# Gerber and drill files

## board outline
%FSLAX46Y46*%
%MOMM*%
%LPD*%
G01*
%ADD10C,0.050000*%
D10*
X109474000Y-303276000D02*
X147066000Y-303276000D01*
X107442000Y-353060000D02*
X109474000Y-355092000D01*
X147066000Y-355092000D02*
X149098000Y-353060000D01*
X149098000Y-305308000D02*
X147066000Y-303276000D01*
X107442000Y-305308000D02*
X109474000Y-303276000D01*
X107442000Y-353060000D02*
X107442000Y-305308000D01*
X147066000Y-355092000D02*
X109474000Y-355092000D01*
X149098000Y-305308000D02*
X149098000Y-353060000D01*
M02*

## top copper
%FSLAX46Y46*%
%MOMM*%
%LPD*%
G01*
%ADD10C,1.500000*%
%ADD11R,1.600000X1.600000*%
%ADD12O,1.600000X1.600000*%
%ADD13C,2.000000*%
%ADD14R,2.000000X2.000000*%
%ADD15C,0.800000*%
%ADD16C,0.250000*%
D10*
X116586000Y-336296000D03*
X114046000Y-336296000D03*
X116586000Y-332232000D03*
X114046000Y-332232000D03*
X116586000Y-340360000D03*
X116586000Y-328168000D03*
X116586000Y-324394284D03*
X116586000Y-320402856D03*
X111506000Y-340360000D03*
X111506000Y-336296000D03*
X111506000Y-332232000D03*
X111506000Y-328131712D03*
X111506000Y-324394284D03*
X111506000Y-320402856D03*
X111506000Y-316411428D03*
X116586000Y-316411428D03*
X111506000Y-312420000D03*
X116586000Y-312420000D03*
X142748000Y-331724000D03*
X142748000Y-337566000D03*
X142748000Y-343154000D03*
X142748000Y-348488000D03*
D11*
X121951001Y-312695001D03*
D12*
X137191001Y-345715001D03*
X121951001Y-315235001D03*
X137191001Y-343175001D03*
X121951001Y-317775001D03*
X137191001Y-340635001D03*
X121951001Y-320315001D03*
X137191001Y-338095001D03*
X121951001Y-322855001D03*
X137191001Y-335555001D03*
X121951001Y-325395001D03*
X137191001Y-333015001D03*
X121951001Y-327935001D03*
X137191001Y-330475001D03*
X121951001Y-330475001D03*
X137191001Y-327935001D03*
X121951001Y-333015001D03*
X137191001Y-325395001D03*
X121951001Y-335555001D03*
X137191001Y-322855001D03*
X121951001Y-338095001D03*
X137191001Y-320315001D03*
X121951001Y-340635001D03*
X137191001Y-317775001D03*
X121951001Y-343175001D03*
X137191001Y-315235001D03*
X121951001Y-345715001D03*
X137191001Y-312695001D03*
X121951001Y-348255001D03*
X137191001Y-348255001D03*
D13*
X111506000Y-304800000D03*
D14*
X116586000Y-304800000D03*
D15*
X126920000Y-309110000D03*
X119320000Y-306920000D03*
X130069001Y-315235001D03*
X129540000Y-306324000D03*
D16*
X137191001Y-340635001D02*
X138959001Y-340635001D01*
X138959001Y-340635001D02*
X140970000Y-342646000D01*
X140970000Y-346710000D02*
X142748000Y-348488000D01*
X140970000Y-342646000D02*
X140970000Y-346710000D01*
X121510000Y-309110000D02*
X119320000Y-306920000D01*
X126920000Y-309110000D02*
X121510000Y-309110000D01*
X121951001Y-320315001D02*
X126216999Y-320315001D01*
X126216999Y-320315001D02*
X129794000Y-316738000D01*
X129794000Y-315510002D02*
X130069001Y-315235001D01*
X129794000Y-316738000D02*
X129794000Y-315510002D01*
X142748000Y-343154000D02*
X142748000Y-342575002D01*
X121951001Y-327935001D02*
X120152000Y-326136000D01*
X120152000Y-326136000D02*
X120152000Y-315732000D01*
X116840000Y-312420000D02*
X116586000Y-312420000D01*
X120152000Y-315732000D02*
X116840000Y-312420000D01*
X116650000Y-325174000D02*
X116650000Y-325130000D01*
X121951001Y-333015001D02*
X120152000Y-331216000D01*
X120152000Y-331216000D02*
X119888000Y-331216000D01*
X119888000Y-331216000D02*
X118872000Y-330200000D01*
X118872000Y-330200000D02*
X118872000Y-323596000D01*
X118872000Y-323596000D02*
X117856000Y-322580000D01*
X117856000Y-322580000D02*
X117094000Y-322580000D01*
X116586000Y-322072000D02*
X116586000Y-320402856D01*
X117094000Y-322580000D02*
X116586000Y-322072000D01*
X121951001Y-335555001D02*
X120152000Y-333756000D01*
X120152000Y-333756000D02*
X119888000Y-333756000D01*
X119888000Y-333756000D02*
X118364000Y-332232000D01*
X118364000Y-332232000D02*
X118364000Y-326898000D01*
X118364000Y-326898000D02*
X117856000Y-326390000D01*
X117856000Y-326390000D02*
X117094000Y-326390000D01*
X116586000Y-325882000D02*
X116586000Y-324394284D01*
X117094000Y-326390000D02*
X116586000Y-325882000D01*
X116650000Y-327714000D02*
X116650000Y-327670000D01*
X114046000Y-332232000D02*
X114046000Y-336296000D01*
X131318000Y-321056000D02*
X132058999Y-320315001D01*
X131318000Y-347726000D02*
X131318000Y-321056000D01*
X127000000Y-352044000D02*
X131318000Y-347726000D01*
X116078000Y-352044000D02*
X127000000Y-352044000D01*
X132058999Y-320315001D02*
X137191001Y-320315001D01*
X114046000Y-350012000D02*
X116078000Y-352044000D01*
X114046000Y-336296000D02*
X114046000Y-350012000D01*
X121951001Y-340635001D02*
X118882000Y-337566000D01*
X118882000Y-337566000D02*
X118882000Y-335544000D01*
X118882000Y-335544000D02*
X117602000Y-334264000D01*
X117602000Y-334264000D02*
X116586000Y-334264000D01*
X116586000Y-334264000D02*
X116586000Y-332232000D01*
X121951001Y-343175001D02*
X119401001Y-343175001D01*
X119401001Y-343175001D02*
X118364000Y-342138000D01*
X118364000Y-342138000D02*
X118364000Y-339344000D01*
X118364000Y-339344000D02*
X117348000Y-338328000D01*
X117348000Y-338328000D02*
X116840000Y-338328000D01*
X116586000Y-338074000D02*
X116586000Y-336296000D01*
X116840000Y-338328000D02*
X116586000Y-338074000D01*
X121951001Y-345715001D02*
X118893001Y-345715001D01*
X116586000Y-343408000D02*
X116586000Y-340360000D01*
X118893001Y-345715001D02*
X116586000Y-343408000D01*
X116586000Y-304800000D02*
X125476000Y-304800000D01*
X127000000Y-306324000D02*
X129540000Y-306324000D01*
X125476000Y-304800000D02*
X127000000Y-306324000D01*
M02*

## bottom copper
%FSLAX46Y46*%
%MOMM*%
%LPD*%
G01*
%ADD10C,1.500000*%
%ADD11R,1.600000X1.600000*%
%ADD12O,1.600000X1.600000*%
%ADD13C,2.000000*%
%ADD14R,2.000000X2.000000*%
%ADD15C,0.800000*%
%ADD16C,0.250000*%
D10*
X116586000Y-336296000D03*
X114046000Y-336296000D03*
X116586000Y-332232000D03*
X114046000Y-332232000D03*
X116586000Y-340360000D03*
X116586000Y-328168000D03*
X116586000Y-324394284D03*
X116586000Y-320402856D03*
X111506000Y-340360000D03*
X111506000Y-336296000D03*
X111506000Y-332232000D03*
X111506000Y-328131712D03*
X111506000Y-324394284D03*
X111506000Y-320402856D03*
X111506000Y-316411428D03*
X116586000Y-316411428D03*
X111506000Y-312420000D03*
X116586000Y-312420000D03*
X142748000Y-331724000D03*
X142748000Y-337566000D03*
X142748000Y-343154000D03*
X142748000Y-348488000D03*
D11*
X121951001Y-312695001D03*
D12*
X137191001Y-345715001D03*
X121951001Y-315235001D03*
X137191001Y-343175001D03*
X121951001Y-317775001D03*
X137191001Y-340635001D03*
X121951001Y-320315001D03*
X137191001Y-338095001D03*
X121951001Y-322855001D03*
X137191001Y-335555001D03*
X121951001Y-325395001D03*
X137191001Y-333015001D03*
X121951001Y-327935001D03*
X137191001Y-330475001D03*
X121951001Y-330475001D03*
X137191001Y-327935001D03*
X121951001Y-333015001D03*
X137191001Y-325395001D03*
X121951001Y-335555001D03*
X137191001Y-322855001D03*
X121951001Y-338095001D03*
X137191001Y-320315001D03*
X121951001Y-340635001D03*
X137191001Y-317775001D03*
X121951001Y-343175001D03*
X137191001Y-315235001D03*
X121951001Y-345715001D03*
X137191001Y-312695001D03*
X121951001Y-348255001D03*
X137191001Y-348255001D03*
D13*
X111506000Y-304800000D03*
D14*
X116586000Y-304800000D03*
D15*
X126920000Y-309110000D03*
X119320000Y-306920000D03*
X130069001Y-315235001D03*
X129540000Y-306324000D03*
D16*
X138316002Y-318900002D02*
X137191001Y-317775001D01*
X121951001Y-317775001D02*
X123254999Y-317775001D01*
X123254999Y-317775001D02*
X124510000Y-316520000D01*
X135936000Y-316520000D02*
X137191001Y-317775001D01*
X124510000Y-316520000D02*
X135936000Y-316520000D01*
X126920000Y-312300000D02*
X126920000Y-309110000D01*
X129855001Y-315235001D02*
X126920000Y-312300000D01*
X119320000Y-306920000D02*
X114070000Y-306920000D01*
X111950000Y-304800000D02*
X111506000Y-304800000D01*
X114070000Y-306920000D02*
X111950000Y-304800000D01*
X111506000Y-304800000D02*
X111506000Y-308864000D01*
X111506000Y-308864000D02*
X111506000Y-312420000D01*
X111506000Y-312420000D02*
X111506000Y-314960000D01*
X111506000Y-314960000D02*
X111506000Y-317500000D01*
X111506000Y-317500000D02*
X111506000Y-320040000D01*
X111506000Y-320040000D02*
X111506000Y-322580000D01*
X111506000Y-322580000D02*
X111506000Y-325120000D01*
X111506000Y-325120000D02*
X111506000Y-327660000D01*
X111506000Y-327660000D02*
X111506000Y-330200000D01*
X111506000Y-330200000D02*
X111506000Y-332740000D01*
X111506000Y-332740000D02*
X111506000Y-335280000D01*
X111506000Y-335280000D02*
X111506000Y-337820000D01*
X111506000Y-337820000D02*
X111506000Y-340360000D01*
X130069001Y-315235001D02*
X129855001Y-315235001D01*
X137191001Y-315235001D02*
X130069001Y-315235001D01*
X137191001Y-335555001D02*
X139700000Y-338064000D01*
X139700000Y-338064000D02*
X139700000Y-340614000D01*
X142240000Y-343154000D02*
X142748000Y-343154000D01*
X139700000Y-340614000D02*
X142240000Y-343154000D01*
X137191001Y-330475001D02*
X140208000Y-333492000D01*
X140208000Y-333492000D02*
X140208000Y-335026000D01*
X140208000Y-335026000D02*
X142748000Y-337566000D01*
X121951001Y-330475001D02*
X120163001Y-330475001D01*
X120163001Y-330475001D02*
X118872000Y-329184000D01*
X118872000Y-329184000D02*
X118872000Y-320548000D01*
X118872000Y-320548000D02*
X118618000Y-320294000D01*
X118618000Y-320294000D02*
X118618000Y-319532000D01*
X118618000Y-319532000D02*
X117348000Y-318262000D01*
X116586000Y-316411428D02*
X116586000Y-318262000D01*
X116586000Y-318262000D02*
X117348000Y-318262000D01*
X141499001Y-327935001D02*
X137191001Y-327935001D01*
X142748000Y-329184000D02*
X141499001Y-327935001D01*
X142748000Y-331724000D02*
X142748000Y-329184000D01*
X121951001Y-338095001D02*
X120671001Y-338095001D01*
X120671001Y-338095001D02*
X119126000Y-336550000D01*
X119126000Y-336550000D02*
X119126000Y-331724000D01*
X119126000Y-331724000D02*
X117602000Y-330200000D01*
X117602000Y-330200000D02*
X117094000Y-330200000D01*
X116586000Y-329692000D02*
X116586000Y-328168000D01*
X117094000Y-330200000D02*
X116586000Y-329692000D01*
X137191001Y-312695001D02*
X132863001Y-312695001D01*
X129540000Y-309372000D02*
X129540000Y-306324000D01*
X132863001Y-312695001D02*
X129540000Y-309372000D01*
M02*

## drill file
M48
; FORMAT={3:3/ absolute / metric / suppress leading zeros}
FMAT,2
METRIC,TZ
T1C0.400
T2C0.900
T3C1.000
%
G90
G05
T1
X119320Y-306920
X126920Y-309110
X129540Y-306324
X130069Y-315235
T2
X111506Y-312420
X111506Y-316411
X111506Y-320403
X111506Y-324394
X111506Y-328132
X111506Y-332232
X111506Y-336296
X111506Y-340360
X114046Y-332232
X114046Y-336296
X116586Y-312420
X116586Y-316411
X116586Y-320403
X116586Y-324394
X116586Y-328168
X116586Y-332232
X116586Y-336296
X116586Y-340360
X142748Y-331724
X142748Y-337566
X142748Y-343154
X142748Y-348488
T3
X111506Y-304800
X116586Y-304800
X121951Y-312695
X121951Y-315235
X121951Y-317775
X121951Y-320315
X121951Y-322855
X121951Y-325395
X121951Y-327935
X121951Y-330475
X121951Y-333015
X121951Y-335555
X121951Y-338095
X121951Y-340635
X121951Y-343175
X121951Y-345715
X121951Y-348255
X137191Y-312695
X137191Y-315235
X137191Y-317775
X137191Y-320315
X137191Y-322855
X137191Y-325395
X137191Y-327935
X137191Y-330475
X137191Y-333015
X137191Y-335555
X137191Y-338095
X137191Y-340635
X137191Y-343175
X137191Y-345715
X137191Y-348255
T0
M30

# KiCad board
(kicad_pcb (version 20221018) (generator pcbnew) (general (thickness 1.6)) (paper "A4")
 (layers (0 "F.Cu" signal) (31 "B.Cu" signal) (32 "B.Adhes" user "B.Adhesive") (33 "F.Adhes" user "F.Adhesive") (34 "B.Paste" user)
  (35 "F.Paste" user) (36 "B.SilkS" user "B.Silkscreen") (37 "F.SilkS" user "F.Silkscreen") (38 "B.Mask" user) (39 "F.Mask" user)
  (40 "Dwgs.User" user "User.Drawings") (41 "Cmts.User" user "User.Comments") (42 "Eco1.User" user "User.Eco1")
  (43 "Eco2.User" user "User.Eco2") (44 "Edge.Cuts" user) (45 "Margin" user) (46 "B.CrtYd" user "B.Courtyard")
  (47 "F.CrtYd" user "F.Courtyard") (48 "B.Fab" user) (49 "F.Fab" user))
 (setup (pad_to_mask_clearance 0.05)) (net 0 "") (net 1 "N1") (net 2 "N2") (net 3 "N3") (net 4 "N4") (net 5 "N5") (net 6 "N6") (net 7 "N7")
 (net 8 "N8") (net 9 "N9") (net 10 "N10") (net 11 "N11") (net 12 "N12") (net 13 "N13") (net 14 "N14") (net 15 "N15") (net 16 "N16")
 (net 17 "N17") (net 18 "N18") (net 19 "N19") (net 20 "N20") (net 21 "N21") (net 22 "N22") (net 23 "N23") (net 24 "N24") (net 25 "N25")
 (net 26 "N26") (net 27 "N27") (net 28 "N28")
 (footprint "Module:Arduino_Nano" (layer "F.Cu") (at 121.951001 312.695001)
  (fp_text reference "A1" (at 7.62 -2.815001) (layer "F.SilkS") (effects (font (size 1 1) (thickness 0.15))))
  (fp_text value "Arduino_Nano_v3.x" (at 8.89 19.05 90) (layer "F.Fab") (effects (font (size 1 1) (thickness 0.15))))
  (pad "1" thru_hole rect (at 0 0) (size 1.6 1.6) (drill 1) (layers "*.Cu" "*.Mask") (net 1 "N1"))
  (pad "2" thru_hole oval (at 0 2.54) (size 1.6 1.6) (drill 1) (layers "*.Cu" "*.Mask") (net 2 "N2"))
  (pad "3" thru_hole oval (at 0 5.08) (size 1.6 1.6) (drill 1) (layers "*.Cu" "*.Mask") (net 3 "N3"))
  (pad "4" thru_hole oval (at 0 7.62) (size 1.6 1.6) (drill 1) (layers "*.Cu" "*.Mask") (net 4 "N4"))
  (pad "5" thru_hole oval (at 0 10.16) (size 1.6 1.6) (drill 1) (layers "*.Cu" "*.Mask") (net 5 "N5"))
  (pad "6" thru_hole oval (at 0 12.7) (size 1.6 1.6) (drill 1) (layers "*.Cu" "*.Mask") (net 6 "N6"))
  (pad "7" thru_hole oval (at 0 15.24) (size 1.6 1.6) (drill 1) (layers "*.Cu" "*.Mask") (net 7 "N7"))
  (pad "8" thru_hole oval (at 0 17.78) (size 1.6 1.6) (drill 1) (layers "*.Cu" "*.Mask") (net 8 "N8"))
  (pad "9" thru_hole oval (at 0 20.32) (size 1.6 1.6) (drill 1) (layers "*.Cu" "*.Mask") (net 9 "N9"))
  (pad "10" thru_hole oval (at 0 22.86) (size 1.6 1.6) (drill 1) (layers "*.Cu" "*.Mask") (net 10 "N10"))
  (pad "11" thru_hole oval (at 0 25.4) (size 1.6 1.6) (drill 1) (layers "*.Cu" "*.Mask") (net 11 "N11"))
  (pad "12" thru_hole oval (at 0 27.94) (size 1.6 1.6) (drill 1) (layers "*.Cu" "*.Mask") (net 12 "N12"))
  (pad "13" thru_hole oval (at 0 30.48) (size 1.6 1.6) (drill 1) (layers "*.Cu" "*.Mask") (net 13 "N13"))
  (pad "14" thru_hole oval (at 0 33.02) (size 1.6 1.6) (drill 1) (layers "*.Cu" "*.Mask") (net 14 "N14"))
  (pad "15" thru_hole oval (at 0 35.56) (size 1.6 1.6) (drill 1) (layers "*.Cu" "*.Mask") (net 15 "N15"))
  (pad "16" thru_hole oval (at 15.24 35.56) (size 1.6 1.6) (drill 1) (layers "*.Cu" "*.Mask") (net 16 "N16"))
  (pad "17" thru_hole oval (at 15.24 33.02) (size 1.6 1.6) (drill 1) (layers "*.Cu" "*.Mask") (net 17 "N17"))
  (pad "18" thru_hole oval (at 15.24 30.48) (size 1.6 1.6) (drill 1) (layers "*.Cu" "*.Mask") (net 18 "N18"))
  (pad "19" thru_hole oval (at 15.24 27.94) (size 1.6 1.6) (drill 1) (layers "*.Cu" "*.Mask") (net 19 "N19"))
  (pad "20" thru_hole oval (at 15.24 25.4) (size 1.6 1.6) (drill 1) (layers "*.Cu" "*.Mask") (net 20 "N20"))
  (pad "21" thru_hole oval (at 15.24 22.86) (size 1.6 1.6) (drill 1) (layers "*.Cu" "*.Mask") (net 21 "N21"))
  (pad "22" thru_hole oval (at 15.24 20.32) (size 1.6 1.6) (drill 1) (layers "*.Cu" "*.Mask") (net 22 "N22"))
  (pad "23" thru_hole oval (at 15.24 17.78) (size 1.6 1.6) (drill 1) (layers "*.Cu" "*.Mask") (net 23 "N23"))
  (pad "24" thru_hole oval (at 15.24 15.24) (size 1.6 1.6) (drill 1) (layers "*.Cu" "*.Mask") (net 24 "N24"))
  (pad "25" thru_hole oval (at 15.24 12.7) (size 1.6 1.6) (drill 1) (layers "*.Cu" "*.Mask") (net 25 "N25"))
  (pad "26" thru_hole oval (at 15.24 10.16) (size 1.6 1.6) (drill 1) (layers "*.Cu" "*.Mask") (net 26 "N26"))
  (pad "27" thru_hole oval (at 15.24 7.62) (size 1.6 1.6) (drill 1) (layers "*.Cu" "*.Mask") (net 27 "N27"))
  (pad "28" thru_hole oval (at 15.24 5.08) (size 1.6 1.6) (drill 1) (layers "*.Cu" "*.Mask") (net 3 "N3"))
  (pad "29" thru_hole oval (at 15.24 2.54) (size 1.6 1.6) (drill 1) (layers "*.Cu" "*.Mask") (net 4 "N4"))
  (pad "30" thru_hole oval (at 15.24 0) (size 1.6 1.6) (drill 1) (layers "*.Cu" "*.Mask") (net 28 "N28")))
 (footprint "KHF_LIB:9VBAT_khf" (layer "F.Cu") (at 111.506 304.8)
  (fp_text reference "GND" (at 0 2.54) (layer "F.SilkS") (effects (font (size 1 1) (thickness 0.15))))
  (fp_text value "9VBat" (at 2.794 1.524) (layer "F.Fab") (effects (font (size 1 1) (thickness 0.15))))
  (pad "1" thru_hole circle (at 0 0) (size 2 2) (drill 1) (layers "*.Cu" "*.Mask") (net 4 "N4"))
  (pad "2" thru_hole rect (at 5.08 0) (size 2 2) (drill 1) (layers "*.Cu" "*.Mask") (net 28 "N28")))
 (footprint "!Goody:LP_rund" (layer "F.Cu") (at 142.748 348.488)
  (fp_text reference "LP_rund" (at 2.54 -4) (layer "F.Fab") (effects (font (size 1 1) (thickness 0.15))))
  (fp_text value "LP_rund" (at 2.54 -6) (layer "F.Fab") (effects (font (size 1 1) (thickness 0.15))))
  (pad "1" thru_hole circle (at 0 0) (size 1.5 1.5) (drill 0.9) (layers "*.Cu" "*.Mask") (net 19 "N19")))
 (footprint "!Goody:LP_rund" (layer "F.Cu") (at 116.586 336.296)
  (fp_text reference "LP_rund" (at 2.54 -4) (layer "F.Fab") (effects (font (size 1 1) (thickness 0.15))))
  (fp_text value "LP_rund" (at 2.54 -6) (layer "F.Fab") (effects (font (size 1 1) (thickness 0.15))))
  (pad "1" thru_hole circle (at 0 0) (size 1.5 1.5) (drill 0.9) (layers "*.Cu" "*.Mask") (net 13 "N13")))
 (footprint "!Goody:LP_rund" (layer "F.Cu") (at 111.506 312.42)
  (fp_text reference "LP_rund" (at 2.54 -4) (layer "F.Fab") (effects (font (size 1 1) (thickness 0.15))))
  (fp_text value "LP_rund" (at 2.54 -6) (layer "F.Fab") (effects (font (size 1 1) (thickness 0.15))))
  (pad "1" thru_hole circle (at 0 0) (size 1.5 1.5) (drill 0.9) (layers "*.Cu" "*.Mask") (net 4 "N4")))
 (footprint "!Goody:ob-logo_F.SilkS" (layer "F.Cu") (at 130.048 329.692 90)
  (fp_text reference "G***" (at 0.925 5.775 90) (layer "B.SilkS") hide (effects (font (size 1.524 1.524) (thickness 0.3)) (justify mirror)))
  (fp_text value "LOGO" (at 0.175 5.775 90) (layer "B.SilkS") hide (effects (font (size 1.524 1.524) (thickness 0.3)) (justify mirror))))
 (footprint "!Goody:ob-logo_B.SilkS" (layer "F.Cu") (at 146.05 323.596 90)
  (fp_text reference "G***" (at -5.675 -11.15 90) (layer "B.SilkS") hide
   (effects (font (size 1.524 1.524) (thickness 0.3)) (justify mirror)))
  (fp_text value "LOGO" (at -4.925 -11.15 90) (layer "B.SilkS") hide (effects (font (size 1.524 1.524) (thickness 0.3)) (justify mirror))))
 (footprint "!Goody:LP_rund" (layer "F.Cu") (at 142.748 343.154)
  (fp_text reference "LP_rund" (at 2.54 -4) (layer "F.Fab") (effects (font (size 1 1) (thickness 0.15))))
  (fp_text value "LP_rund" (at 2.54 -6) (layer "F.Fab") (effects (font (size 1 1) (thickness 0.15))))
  (pad "1" thru_hole circle (at 0 0) (size 1.5 1.5) (drill 0.9) (layers "*.Cu" "*.Mask") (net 21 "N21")))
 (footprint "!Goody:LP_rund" (layer "F.Cu") (at 111.506 340.36)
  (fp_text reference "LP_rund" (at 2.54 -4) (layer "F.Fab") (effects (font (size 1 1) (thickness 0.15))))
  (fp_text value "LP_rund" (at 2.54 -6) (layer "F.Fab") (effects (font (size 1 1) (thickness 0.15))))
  (pad "1" thru_hole circle (at 0 0) (size 1.5 1.5) (drill 0.9) (layers "*.Cu" "*.Mask") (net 4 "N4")))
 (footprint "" (layer "F.Cu") (at 112.268 348.488)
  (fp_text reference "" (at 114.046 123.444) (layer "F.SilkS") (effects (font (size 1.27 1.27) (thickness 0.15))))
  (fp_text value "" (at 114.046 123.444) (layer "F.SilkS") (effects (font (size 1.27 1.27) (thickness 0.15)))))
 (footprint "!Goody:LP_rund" (layer "F.Cu") (at 116.586 312.42)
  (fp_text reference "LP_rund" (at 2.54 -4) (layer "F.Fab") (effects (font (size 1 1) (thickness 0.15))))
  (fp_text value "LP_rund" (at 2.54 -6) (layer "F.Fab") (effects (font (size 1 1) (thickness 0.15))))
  (pad "1" thru_hole circle (at 0 0) (size 1.5 1.5) (drill 0.9) (layers "*.Cu" "*.Mask") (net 7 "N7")))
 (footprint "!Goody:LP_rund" (layer "F.Cu") (at 116.586 332.232)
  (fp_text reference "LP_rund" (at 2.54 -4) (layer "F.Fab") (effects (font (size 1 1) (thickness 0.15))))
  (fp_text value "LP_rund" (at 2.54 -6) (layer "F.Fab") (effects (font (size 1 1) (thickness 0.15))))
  (pad "1" thru_hole circle (at 0 0) (size 1.5 1.5) (drill 0.9) (layers "*.Cu" "*.Mask") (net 12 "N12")))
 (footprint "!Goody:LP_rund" (layer "F.Cu") (at 116.586 340.36)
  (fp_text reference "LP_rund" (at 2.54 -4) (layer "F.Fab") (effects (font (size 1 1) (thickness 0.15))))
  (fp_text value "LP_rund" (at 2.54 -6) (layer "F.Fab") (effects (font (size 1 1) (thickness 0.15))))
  (pad "1" thru_hole circle (at 0 0) (size 1.5 1.5) (drill 0.9) (layers "*.Cu" "*.Mask") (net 14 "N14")))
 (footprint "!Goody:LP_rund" (layer "F.Cu") (at 111.506 335.13486)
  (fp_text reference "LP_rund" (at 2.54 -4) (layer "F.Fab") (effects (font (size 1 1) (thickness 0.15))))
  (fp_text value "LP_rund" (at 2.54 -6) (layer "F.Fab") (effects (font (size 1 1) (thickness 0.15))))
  (pad "1" thru_hole circle (at 0 -2.90286) (size 1.5 1.5) (drill 0.9) (layers "*.Cu" "*.Mask") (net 4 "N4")))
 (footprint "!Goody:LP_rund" (layer "F.Cu") (at 111.506 330.2)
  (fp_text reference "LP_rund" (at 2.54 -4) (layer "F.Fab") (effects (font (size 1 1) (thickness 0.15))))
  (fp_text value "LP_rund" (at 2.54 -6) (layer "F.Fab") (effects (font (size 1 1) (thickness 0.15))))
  (pad "1" thru_hole circle (at 0 -5.805716) (size 1.5 1.5) (drill 0.9) (layers "*.Cu" "*.Mask") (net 4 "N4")))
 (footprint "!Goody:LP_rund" (layer "F.Cu") (at 116.586 325.12)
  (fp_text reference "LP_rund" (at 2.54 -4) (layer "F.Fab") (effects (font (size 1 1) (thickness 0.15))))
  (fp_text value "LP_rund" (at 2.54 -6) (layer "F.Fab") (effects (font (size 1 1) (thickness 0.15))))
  (pad "1" thru_hole circle (at 0 -8.708572) (size 1.5 1.5) (drill 0.9) (layers "*.Cu" "*.Mask") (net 8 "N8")))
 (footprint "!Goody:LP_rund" (layer "F.Cu") (at 142.748 331.724)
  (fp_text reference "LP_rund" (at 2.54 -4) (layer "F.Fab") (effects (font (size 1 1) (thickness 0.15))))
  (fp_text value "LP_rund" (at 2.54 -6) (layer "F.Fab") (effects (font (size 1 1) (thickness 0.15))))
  (pad "1" thru_hole circle (at 0 0) (size 1.5 1.5) (drill 0.9) (layers "*.Cu" "*.Mask") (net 24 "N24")))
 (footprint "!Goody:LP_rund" (layer "F.Cu") (at 111.506 336.296)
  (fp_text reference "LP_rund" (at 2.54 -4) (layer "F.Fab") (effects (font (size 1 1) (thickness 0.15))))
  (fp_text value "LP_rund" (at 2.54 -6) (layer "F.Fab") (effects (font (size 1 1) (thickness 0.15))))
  (pad "1" thru_hole circle (at 0 0) (size 1.5 1.5) (drill 0.9) (layers "*.Cu" "*.Mask") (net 4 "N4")))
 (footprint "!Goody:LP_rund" (layer "F.Cu") (at 116.586 324.394284)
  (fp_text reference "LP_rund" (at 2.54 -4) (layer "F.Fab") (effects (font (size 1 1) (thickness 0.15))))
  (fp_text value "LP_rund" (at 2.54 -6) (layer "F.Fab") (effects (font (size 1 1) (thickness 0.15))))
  (pad "1" thru_hole circle (at 0 0) (size 1.5 1.5) (drill 0.9) (layers "*.Cu" "*.Mask") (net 10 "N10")))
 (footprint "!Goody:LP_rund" (layer "F.Cu") (at 116.586 327.66)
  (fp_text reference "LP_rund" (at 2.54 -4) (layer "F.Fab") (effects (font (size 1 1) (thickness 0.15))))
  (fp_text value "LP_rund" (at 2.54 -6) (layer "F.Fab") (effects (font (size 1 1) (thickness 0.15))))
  (pad "1" thru_hole circle (at 0 -7.257144) (size 1.5 1.5) (drill 0.9) (layers "*.Cu" "*.Mask") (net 9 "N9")))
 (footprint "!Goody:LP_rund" (layer "F.Cu") (at 116.586 328.168)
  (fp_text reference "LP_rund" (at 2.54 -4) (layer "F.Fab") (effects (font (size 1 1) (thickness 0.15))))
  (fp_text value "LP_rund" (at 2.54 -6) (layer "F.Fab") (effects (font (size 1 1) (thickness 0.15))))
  (pad "1" thru_hole circle (at 0 0) (size 1.5 1.5) (drill 0.9) (layers "*.Cu" "*.Mask") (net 11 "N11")))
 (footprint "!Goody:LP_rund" (layer "F.Cu") (at 114.046 336.296)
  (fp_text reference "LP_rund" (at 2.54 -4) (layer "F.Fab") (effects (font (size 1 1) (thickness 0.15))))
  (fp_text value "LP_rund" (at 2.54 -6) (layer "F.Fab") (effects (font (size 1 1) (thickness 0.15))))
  (pad "1" thru_hole circle (at 0 0) (size 1.5 1.5) (drill 0.9) (layers "*.Cu" "*.Mask") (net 27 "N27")))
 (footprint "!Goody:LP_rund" (layer "F.Cu") (at 114.046 332.232)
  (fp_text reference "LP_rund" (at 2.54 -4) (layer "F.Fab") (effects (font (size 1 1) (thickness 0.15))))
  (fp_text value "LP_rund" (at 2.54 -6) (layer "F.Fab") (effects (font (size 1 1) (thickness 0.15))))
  (pad "1" thru_hole circle (at 0 0) (size 1.5 1.5) (drill 0.9) (layers "*.Cu" "*.Mask") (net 27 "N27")))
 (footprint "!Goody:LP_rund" (layer "F.Cu") (at 111.506 327.66)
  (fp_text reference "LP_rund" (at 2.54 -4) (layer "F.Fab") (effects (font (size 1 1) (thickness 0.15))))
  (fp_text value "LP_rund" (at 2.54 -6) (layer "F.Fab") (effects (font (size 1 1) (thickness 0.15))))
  (pad "1" thru_hole circle (at 0 -7.257144) (size 1.5 1.5) (drill 0.9) (layers "*.Cu" "*.Mask") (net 4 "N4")))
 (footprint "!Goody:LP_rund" (layer "F.Cu") (at 111.506 332.486)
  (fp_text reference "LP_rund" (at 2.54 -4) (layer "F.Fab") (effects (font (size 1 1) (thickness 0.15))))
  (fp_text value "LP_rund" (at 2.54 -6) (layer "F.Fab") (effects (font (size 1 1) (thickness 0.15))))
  (pad "1" thru_hole circle (at 0 -4.354288) (size 1.5 1.5) (drill 0.9) (layers "*.Cu" "*.Mask") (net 4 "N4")))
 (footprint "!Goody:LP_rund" (layer "F.Cu") (at 111.506 318.008)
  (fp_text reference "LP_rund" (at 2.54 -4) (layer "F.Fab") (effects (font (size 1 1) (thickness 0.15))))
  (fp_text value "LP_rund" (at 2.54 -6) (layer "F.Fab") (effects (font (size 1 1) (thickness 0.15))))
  (pad "1" thru_hole circle (at 0 -1.596572) (size 1.5 1.5) (drill 0.9) (layers "*.Cu" "*.Mask") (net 4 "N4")))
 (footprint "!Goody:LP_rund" (layer "F.Cu") (at 142.748 337.566)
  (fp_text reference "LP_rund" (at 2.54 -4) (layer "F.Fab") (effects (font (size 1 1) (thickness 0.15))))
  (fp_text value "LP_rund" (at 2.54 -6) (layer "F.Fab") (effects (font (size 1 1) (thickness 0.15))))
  (pad "1" thru_hole circle (at 0 0) (size 1.5 1.5) (drill 0.9) (layers "*.Cu" "*.Mask") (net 23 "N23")))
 (gr_line (start 107.442 353.06) (end 107.442 305.308) (stroke (width 0.05) (type solid)) (layer "Edge.Cuts"))
 (gr_line (start 109.474 303.276) (end 147.066 303.276) (stroke (width 0.05) (type solid)) (layer "Edge.Cuts"))
 (gr_line (start 147.066 355.092) (end 109.474 355.092) (stroke (width 0.05) (type solid)) (layer "Edge.Cuts"))
 (gr_line (start 147.066 355.092) (end 149.098 353.06) (stroke (width 0.05) (type solid)) (layer "Edge.Cuts"))
 (gr_line (start 149.098 305.308) (end 147.066 303.276) (stroke (width 0.05) (type solid)) (layer "Edge.Cuts"))
 (gr_line (start 149.098 305.308) (end 149.098 353.06) (stroke (width 0.05) (type solid)) (layer "Edge.Cuts"))
 (gr_line (start 107.442 305.308) (end 109.474 303.276) (stroke (width 0.05) (type solid)) (layer "Edge.Cuts"))
 (gr_line (start 107.442 353.06) (end 109.474 355.092) (stroke (width 0.05) (type solid)) (layer "Edge.Cuts"))
 (segment (start 135.936 316.52) (end 137.191001 317.775001) (width 0.25) (layer "B.Cu") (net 3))
 (segment (start 124.51 316.52) (end 135.936 316.52) (width 0.25) (layer "B.Cu") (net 3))
 (segment (start 123.254999 317.775001) (end 124.51 316.52) (width 0.25) (layer "B.Cu") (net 3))
 (segment (start 138.316002 318.900002) (end 137.191001 317.775001) (width 0.25) (layer "B.Cu") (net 3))
 (segment (start 121.951001 317.775001) (end 123.254999 317.775001) (width 0.25) (layer "B.Cu") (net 3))
 (segment (start 137.191001 340.635001) (end 138.959001 340.635001) (width 0.25) (layer "F.Cu") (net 19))
 (segment (start 140.97 346.71) (end 142.748 348.488) (width 0.25) (layer "F.Cu") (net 19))
 (segment (start 138.959001 340.635001) (end 140.97 342.646) (width 0.25) (layer "F.Cu") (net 19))
 (segment (start 140.97 342.646) (end 140.97 346.71) (width 0.25) (layer "F.Cu") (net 19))
 (segment (start 129.794 315.510002) (end 130.069001 315.235001) (width 0.25) (layer "F.Cu") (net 4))
 (segment (start 121.951001 320.315001) (end 126.216999 320.315001) (width 0.25) (layer "F.Cu") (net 4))
 (segment (start 129.794 316.738) (end 129.794 315.510002) (width 0.25) (layer "F.Cu") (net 4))
 (segment (start 126.216999 320.315001) (end 129.794 316.738) (width 0.25) (layer "F.Cu") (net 4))
 (segment (start 121.51 309.11) (end 119.32 306.92) (width 0.25) (layer "F.Cu") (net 4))
 (segment (start 126.92 309.11) (end 121.51 309.11) (width 0.25) (layer "F.Cu") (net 4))
 (via (at 119.32 306.92) (size 0.8) (drill 0.4) (layers "F.Cu" "B.Cu") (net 4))
 (via (at 130.069001 315.235001) (size 0.8) (drill 0.4) (layers "F.Cu" "B.Cu") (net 4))
 (via (at 126.92 309.11) (size 0.8) (drill 0.4) (layers "F.Cu" "B.Cu") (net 4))
 (segment (start 129.855001 315.235001) (end 126.92 312.3) (width 0.25) (layer "B.Cu") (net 4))
 (segment (start 111.506 330.2) (end 111.506 332.74) (width 0.25) (layer "B.Cu") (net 4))
 (segment (start 111.506 325.12) (end 111.506 327.66) (width 0.25) (layer "B.Cu") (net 4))
 (segment (start 111.506 312.42) (end 111.506 314.96) (width 0.25) (layer "B.Cu") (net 4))
 (segment (start 111.95 304.8) (end 111.506 304.8) (width 0.25) (layer "B.Cu") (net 4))
 (segment (start 130.069001 315.235001) (end 129.855001 315.235001) (width 0.25) (layer "B.Cu") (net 4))
 (segment (start 111.506 317.5) (end 111.506 320.04) (width 0.25) (layer "B.Cu") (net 4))
 (segment (start 111.506 327.66) (end 111.506 330.2) (width 0.25) (layer "B.Cu") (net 4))
 (segment (start 126.92 312.3) (end 126.92 309.11) (width 0.25) (layer "B.Cu") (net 4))
 (segment (start 111.506 308.864) (end 111.506 312.42) (width 0.25) (layer "B.Cu") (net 4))
 (segment (start 119.32 306.92) (end 114.07 306.92) (width 0.25) (layer "B.Cu") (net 4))
 (segment (start 111.506 332.74) (end 111.506 335.28) (width 0.25) (layer "B.Cu") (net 4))
 (segment (start 111.506 304.8) (end 111.506 308.864) (width 0.25) (layer "B.Cu") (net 4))
 (segment (start 137.191001 315.235001) (end 130.069001 315.235001) (width 0.25) (layer "B.Cu") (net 4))
 (segment (start 114.07 306.92) (end 111.95 304.8) (width 0.25) (layer "B.Cu") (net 4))
 (segment (start 111.506 314.96) (end 111.506 317.5) (width 0.25) (layer "B.Cu") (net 4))
 (segment (start 111.506 337.82) (end 111.506 340.36) (width 0.25) (layer "B.Cu") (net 4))
 (segment (start 111.506 320.04) (end 111.506 322.58) (width 0.25) (layer "B.Cu") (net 4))
 (segment (start 111.506 322.58) (end 111.506 325.12) (width 0.25) (layer "B.Cu") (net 4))
 (segment (start 111.506 335.28) (end 111.506 337.82) (width 0.25) (layer "B.Cu") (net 4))
 (segment (start 142.748 343.154) (end 142.748 342.575002) (width 0.25) (layer "F.Cu") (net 21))
 (segment (start 137.191001 335.555001) (end 139.7 338.064) (width 0.25) (layer "B.Cu") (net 21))
 (segment (start 139.7 340.614) (end 142.24 343.154) (width 0.25) (layer "B.Cu") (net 21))
 (segment (start 142.24 343.154) (end 142.748 343.154) (width 0.25) (layer "B.Cu") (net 21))
 (segment (start 139.7 338.064) (end 139.7 340.614) (width 0.25) (layer "B.Cu") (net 21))
 (segment (start 120.152 315.732) (end 116.84 312.42) (width 0.25) (layer "F.Cu") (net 7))
 (segment (start 120.152 326.136) (end 120.152 315.732) (width 0.25) (layer "F.Cu") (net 7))
 (segment (start 121.951001 327.935001) (end 120.152 326.136) (width 0.25) (layer "F.Cu") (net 7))
 (segment (start 116.84 312.42) (end 116.586 312.42) (width 0.25) (layer "F.Cu") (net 7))
 (segment (start 140.208 333.492) (end 140.208 335.026) (width 0.25) (layer "B.Cu") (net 23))
 (segment (start 140.208 335.026) (end 142.748 337.566) (width 0.25) (layer "B.Cu") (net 23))
 (segment (start 137.191001 330.475001) (end 140.208 333.492) (width 0.25) (layer "B.Cu") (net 23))
 (segment (start 118.872 329.184) (end 118.872 320.548) (width 0.25) (layer "B.Cu") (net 8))
 (segment (start 118.872 320.548) (end 118.618 320.294) (width 0.25) (layer "B.Cu") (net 8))
 (segment (start 118.618 320.294) (end 118.618 319.532) (width 0.25) (layer "B.Cu") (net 8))
 (segment (start 116.586 316.411428) (end 116.586 318.262) (width 0.25) (layer "B.Cu") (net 8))
 (segment (start 118.618 319.532) (end 117.348 318.262) (width 0.25) (layer "B.Cu") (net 8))
 (segment (start 121.951001 330.475001) (end 120.163001 330.475001) (width 0.25) (layer "B.Cu") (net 8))
 (segment (start 120.163001 330.475001) (end 118.872 329.184) (width 0.25) (layer "B.Cu") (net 8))
 (segment (start 116.586 318.262) (end 117.348 318.262) (width 0.25) (layer "B.Cu") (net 8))
 (segment (start 142.748 331.724) (end 142.748 329.184) (width 0.25) (layer "B.Cu") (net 24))
 (segment (start 141.499001 327.935001) (end 137.191001 327.935001) (width 0.25) (layer "B.Cu") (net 24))
 (segment (start 142.748 329.184) (end 141.499001 327.935001) (width 0.25) (layer "B.Cu") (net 24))
 (segment (start 118.872 323.596) (end 117.856 322.58) (width 0.25) (layer "F.Cu") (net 9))
 (segment (start 120.152 331.216) (end 119.888 331.216) (width 0.25) (layer "F.Cu") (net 9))
 (segment (start 117.856 322.58) (end 117.094 322.58) (width 0.25) (layer "F.Cu") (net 9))
 (segment (start 121.951001 333.015001) (end 120.152 331.216) (width 0.25) (layer "F.Cu") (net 9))
 (segment (start 118.872 330.2) (end 118.872 323.596) (width 0.25) (layer "F.Cu") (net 9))
 (segment (start 117.094 322.58) (end 116.586 322.072) (width 0.25) (layer "F.Cu") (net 9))
 (segment (start 116.586 322.072) (end 116.586 320.402856) (width 0.25) (layer "F.Cu") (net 9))
 (segment (start 119.888 331.216) (end 118.872 330.2) (width 0.25) (layer "F.Cu") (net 9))
 (segment (start 118.364 332.232) (end 118.364 326.898) (width 0.25) (layer "F.Cu") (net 10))
 (segment (start 121.951001 335.555001) (end 120.152 333.756) (width 0.25) (layer "F.Cu") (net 10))
 (segment (start 118.364 326.898) (end 117.856 326.39) (width 0.25) (layer "F.Cu") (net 10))
 (segment (start 116.65 325.174) (end 116.65 325.13) (width 0.25) (layer "F.Cu") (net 10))
 (segment (start 119.888 333.756) (end 118.364 332.232) (width 0.25) (layer "F.Cu") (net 10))
 (segment (start 116.586 325.882) (end 116.586 324.394284) (width 0.25) (layer "F.Cu") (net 10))
 (segment (start 117.856 326.39) (end 117.094 326.39) (width 0.25) (layer "F.Cu") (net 10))
 (segment (start 117.094 326.39) (end 116.586 325.882) (width 0.25) (layer "F.Cu") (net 10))
 (segment (start 120.152 333.756) (end 119.888 333.756) (width 0.25) (layer "F.Cu") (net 10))
 (segment (start 116.65 327.714) (end 116.65 327.67) (width 0.25) (layer "F.Cu") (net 11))
 (segment (start 117.094 330.2) (end 116.586 329.692) (width 0.25) (layer "B.Cu") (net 11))
 (segment (start 117.602 330.2) (end 117.094 330.2) (width 0.25) (layer "B.Cu") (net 11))
 (segment (start 121.951001 338.095001) (end 120.671001 338.095001) (width 0.25) (layer "B.Cu") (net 11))
 (segment (start 116.586 329.692) (end 116.586 328.168) (width 0.25) (layer "B.Cu") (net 11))
 (segment (start 120.671001 338.095001) (end 119.126 336.55) (width 0.25) (layer "B.Cu") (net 11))
 (segment (start 119.126 336.55) (end 119.126 331.724) (width 0.25) (layer "B.Cu") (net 11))
 (segment (start 119.126 331.724) (end 117.602 330.2) (width 0.25) (layer "B.Cu") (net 11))
 (segment (start 131.318 321.056) (end 132.058999 320.315001) (width 0.25) (layer "F.Cu") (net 27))
 (segment (start 114.046 336.296) (end 114.046 350.012) (width 0.25) (layer "F.Cu") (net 27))
 (segment (start 116.078 352.044) (end 127 352.044) (width 0.25) (layer "F.Cu") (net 27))
 (segment (start 114.046 332.232) (end 114.046 336.296) (width 0.25) (layer "F.Cu") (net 27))
 (segment (start 131.318 347.726) (end 131.318 321.056) (width 0.25) (layer "F.Cu") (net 27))
 (segment (start 114.046 350.012) (end 116.078 352.044) (width 0.25) (layer "F.Cu") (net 27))
 (segment (start 127 352.044) (end 131.318 347.726) (width 0.25) (layer "F.Cu") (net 27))
 (segment (start 132.058999 320.315001) (end 137.191001 320.315001) (width 0.25) (layer "F.Cu") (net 27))
 (segment (start 121.951001 340.635001) (end 118.882 337.566) (width 0.25) (layer "F.Cu") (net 12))
 (segment (start 118.882 337.566) (end 118.882 335.544) (width 0.25) (layer "F.Cu") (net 12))
 (segment (start 118.882 335.544) (end 117.602 334.264) (width 0.25) (layer "F.Cu") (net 12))
 (segment (start 116.586 334.264) (end 116.586 332.232) (width 0.25) (layer "F.Cu") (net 12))
 (segment (start 117.602 334.264) (end 116.586 334.264) (width 0.25) (layer "F.Cu") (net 12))
 (segment (start 121.951001 343.175001) (end 119.401001 343.175001) (width 0.25) (layer "F.Cu") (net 13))
 (segment (start 116.84 338.328) (end 116.586 338.074) (width 0.25) (layer "F.Cu") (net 13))
 (segment (start 116.586 338.074) (end 116.586 336.296) (width 0.25) (layer "F.Cu") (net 13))
 (segment (start 118.364 342.138) (end 118.364 339.344) (width 0.25) (layer "F.Cu") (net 13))
 (segment (start 119.401001 343.175001) (end 118.364 342.138) (width 0.25) (layer "F.Cu") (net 13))
 (segment (start 118.364 339.344) (end 117.348 338.328) (width 0.25) (layer "F.Cu") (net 13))
 (segment (start 117.348 338.328) (end 116.84 338.328) (width 0.25) (layer "F.Cu") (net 13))
 (segment (start 116.586 343.408) (end 116.586 340.36) (width 0.25) (layer "F.Cu") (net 14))
 (segment (start 118.893001 345.715001) (end 116.586 343.408) (width 0.25) (layer "F.Cu") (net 14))
 (segment (start 121.951001 345.715001) (end 118.893001 345.715001) (width 0.25) (layer "F.Cu") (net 14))
 (segment (start 125.476 304.8) (end 127 306.324) (width 0.25) (layer "F.Cu") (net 28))
 (segment (start 127 306.324) (end 129.54 306.324) (width 0.25) (layer "F.Cu") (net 28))
 (segment (start 116.586 304.8) (end 125.476 304.8) (width 0.25) (layer "F.Cu") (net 28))
 (via (at 129.54 306.324) (size 0.8) (drill 0.4) (layers "F.Cu" "B.Cu") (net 28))
 (segment (start 132.863001 312.695001) (end 129.54 309.372) (width 0.25) (layer "B.Cu") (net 28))
 (segment (start 129.54 309.372) (end 129.54 306.324) (width 0.25) (layer "B.Cu") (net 28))
 (segment (start 137.191001 312.695001) (end 132.863001 312.695001) (width 0.25) (layer "B.Cu") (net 28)))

